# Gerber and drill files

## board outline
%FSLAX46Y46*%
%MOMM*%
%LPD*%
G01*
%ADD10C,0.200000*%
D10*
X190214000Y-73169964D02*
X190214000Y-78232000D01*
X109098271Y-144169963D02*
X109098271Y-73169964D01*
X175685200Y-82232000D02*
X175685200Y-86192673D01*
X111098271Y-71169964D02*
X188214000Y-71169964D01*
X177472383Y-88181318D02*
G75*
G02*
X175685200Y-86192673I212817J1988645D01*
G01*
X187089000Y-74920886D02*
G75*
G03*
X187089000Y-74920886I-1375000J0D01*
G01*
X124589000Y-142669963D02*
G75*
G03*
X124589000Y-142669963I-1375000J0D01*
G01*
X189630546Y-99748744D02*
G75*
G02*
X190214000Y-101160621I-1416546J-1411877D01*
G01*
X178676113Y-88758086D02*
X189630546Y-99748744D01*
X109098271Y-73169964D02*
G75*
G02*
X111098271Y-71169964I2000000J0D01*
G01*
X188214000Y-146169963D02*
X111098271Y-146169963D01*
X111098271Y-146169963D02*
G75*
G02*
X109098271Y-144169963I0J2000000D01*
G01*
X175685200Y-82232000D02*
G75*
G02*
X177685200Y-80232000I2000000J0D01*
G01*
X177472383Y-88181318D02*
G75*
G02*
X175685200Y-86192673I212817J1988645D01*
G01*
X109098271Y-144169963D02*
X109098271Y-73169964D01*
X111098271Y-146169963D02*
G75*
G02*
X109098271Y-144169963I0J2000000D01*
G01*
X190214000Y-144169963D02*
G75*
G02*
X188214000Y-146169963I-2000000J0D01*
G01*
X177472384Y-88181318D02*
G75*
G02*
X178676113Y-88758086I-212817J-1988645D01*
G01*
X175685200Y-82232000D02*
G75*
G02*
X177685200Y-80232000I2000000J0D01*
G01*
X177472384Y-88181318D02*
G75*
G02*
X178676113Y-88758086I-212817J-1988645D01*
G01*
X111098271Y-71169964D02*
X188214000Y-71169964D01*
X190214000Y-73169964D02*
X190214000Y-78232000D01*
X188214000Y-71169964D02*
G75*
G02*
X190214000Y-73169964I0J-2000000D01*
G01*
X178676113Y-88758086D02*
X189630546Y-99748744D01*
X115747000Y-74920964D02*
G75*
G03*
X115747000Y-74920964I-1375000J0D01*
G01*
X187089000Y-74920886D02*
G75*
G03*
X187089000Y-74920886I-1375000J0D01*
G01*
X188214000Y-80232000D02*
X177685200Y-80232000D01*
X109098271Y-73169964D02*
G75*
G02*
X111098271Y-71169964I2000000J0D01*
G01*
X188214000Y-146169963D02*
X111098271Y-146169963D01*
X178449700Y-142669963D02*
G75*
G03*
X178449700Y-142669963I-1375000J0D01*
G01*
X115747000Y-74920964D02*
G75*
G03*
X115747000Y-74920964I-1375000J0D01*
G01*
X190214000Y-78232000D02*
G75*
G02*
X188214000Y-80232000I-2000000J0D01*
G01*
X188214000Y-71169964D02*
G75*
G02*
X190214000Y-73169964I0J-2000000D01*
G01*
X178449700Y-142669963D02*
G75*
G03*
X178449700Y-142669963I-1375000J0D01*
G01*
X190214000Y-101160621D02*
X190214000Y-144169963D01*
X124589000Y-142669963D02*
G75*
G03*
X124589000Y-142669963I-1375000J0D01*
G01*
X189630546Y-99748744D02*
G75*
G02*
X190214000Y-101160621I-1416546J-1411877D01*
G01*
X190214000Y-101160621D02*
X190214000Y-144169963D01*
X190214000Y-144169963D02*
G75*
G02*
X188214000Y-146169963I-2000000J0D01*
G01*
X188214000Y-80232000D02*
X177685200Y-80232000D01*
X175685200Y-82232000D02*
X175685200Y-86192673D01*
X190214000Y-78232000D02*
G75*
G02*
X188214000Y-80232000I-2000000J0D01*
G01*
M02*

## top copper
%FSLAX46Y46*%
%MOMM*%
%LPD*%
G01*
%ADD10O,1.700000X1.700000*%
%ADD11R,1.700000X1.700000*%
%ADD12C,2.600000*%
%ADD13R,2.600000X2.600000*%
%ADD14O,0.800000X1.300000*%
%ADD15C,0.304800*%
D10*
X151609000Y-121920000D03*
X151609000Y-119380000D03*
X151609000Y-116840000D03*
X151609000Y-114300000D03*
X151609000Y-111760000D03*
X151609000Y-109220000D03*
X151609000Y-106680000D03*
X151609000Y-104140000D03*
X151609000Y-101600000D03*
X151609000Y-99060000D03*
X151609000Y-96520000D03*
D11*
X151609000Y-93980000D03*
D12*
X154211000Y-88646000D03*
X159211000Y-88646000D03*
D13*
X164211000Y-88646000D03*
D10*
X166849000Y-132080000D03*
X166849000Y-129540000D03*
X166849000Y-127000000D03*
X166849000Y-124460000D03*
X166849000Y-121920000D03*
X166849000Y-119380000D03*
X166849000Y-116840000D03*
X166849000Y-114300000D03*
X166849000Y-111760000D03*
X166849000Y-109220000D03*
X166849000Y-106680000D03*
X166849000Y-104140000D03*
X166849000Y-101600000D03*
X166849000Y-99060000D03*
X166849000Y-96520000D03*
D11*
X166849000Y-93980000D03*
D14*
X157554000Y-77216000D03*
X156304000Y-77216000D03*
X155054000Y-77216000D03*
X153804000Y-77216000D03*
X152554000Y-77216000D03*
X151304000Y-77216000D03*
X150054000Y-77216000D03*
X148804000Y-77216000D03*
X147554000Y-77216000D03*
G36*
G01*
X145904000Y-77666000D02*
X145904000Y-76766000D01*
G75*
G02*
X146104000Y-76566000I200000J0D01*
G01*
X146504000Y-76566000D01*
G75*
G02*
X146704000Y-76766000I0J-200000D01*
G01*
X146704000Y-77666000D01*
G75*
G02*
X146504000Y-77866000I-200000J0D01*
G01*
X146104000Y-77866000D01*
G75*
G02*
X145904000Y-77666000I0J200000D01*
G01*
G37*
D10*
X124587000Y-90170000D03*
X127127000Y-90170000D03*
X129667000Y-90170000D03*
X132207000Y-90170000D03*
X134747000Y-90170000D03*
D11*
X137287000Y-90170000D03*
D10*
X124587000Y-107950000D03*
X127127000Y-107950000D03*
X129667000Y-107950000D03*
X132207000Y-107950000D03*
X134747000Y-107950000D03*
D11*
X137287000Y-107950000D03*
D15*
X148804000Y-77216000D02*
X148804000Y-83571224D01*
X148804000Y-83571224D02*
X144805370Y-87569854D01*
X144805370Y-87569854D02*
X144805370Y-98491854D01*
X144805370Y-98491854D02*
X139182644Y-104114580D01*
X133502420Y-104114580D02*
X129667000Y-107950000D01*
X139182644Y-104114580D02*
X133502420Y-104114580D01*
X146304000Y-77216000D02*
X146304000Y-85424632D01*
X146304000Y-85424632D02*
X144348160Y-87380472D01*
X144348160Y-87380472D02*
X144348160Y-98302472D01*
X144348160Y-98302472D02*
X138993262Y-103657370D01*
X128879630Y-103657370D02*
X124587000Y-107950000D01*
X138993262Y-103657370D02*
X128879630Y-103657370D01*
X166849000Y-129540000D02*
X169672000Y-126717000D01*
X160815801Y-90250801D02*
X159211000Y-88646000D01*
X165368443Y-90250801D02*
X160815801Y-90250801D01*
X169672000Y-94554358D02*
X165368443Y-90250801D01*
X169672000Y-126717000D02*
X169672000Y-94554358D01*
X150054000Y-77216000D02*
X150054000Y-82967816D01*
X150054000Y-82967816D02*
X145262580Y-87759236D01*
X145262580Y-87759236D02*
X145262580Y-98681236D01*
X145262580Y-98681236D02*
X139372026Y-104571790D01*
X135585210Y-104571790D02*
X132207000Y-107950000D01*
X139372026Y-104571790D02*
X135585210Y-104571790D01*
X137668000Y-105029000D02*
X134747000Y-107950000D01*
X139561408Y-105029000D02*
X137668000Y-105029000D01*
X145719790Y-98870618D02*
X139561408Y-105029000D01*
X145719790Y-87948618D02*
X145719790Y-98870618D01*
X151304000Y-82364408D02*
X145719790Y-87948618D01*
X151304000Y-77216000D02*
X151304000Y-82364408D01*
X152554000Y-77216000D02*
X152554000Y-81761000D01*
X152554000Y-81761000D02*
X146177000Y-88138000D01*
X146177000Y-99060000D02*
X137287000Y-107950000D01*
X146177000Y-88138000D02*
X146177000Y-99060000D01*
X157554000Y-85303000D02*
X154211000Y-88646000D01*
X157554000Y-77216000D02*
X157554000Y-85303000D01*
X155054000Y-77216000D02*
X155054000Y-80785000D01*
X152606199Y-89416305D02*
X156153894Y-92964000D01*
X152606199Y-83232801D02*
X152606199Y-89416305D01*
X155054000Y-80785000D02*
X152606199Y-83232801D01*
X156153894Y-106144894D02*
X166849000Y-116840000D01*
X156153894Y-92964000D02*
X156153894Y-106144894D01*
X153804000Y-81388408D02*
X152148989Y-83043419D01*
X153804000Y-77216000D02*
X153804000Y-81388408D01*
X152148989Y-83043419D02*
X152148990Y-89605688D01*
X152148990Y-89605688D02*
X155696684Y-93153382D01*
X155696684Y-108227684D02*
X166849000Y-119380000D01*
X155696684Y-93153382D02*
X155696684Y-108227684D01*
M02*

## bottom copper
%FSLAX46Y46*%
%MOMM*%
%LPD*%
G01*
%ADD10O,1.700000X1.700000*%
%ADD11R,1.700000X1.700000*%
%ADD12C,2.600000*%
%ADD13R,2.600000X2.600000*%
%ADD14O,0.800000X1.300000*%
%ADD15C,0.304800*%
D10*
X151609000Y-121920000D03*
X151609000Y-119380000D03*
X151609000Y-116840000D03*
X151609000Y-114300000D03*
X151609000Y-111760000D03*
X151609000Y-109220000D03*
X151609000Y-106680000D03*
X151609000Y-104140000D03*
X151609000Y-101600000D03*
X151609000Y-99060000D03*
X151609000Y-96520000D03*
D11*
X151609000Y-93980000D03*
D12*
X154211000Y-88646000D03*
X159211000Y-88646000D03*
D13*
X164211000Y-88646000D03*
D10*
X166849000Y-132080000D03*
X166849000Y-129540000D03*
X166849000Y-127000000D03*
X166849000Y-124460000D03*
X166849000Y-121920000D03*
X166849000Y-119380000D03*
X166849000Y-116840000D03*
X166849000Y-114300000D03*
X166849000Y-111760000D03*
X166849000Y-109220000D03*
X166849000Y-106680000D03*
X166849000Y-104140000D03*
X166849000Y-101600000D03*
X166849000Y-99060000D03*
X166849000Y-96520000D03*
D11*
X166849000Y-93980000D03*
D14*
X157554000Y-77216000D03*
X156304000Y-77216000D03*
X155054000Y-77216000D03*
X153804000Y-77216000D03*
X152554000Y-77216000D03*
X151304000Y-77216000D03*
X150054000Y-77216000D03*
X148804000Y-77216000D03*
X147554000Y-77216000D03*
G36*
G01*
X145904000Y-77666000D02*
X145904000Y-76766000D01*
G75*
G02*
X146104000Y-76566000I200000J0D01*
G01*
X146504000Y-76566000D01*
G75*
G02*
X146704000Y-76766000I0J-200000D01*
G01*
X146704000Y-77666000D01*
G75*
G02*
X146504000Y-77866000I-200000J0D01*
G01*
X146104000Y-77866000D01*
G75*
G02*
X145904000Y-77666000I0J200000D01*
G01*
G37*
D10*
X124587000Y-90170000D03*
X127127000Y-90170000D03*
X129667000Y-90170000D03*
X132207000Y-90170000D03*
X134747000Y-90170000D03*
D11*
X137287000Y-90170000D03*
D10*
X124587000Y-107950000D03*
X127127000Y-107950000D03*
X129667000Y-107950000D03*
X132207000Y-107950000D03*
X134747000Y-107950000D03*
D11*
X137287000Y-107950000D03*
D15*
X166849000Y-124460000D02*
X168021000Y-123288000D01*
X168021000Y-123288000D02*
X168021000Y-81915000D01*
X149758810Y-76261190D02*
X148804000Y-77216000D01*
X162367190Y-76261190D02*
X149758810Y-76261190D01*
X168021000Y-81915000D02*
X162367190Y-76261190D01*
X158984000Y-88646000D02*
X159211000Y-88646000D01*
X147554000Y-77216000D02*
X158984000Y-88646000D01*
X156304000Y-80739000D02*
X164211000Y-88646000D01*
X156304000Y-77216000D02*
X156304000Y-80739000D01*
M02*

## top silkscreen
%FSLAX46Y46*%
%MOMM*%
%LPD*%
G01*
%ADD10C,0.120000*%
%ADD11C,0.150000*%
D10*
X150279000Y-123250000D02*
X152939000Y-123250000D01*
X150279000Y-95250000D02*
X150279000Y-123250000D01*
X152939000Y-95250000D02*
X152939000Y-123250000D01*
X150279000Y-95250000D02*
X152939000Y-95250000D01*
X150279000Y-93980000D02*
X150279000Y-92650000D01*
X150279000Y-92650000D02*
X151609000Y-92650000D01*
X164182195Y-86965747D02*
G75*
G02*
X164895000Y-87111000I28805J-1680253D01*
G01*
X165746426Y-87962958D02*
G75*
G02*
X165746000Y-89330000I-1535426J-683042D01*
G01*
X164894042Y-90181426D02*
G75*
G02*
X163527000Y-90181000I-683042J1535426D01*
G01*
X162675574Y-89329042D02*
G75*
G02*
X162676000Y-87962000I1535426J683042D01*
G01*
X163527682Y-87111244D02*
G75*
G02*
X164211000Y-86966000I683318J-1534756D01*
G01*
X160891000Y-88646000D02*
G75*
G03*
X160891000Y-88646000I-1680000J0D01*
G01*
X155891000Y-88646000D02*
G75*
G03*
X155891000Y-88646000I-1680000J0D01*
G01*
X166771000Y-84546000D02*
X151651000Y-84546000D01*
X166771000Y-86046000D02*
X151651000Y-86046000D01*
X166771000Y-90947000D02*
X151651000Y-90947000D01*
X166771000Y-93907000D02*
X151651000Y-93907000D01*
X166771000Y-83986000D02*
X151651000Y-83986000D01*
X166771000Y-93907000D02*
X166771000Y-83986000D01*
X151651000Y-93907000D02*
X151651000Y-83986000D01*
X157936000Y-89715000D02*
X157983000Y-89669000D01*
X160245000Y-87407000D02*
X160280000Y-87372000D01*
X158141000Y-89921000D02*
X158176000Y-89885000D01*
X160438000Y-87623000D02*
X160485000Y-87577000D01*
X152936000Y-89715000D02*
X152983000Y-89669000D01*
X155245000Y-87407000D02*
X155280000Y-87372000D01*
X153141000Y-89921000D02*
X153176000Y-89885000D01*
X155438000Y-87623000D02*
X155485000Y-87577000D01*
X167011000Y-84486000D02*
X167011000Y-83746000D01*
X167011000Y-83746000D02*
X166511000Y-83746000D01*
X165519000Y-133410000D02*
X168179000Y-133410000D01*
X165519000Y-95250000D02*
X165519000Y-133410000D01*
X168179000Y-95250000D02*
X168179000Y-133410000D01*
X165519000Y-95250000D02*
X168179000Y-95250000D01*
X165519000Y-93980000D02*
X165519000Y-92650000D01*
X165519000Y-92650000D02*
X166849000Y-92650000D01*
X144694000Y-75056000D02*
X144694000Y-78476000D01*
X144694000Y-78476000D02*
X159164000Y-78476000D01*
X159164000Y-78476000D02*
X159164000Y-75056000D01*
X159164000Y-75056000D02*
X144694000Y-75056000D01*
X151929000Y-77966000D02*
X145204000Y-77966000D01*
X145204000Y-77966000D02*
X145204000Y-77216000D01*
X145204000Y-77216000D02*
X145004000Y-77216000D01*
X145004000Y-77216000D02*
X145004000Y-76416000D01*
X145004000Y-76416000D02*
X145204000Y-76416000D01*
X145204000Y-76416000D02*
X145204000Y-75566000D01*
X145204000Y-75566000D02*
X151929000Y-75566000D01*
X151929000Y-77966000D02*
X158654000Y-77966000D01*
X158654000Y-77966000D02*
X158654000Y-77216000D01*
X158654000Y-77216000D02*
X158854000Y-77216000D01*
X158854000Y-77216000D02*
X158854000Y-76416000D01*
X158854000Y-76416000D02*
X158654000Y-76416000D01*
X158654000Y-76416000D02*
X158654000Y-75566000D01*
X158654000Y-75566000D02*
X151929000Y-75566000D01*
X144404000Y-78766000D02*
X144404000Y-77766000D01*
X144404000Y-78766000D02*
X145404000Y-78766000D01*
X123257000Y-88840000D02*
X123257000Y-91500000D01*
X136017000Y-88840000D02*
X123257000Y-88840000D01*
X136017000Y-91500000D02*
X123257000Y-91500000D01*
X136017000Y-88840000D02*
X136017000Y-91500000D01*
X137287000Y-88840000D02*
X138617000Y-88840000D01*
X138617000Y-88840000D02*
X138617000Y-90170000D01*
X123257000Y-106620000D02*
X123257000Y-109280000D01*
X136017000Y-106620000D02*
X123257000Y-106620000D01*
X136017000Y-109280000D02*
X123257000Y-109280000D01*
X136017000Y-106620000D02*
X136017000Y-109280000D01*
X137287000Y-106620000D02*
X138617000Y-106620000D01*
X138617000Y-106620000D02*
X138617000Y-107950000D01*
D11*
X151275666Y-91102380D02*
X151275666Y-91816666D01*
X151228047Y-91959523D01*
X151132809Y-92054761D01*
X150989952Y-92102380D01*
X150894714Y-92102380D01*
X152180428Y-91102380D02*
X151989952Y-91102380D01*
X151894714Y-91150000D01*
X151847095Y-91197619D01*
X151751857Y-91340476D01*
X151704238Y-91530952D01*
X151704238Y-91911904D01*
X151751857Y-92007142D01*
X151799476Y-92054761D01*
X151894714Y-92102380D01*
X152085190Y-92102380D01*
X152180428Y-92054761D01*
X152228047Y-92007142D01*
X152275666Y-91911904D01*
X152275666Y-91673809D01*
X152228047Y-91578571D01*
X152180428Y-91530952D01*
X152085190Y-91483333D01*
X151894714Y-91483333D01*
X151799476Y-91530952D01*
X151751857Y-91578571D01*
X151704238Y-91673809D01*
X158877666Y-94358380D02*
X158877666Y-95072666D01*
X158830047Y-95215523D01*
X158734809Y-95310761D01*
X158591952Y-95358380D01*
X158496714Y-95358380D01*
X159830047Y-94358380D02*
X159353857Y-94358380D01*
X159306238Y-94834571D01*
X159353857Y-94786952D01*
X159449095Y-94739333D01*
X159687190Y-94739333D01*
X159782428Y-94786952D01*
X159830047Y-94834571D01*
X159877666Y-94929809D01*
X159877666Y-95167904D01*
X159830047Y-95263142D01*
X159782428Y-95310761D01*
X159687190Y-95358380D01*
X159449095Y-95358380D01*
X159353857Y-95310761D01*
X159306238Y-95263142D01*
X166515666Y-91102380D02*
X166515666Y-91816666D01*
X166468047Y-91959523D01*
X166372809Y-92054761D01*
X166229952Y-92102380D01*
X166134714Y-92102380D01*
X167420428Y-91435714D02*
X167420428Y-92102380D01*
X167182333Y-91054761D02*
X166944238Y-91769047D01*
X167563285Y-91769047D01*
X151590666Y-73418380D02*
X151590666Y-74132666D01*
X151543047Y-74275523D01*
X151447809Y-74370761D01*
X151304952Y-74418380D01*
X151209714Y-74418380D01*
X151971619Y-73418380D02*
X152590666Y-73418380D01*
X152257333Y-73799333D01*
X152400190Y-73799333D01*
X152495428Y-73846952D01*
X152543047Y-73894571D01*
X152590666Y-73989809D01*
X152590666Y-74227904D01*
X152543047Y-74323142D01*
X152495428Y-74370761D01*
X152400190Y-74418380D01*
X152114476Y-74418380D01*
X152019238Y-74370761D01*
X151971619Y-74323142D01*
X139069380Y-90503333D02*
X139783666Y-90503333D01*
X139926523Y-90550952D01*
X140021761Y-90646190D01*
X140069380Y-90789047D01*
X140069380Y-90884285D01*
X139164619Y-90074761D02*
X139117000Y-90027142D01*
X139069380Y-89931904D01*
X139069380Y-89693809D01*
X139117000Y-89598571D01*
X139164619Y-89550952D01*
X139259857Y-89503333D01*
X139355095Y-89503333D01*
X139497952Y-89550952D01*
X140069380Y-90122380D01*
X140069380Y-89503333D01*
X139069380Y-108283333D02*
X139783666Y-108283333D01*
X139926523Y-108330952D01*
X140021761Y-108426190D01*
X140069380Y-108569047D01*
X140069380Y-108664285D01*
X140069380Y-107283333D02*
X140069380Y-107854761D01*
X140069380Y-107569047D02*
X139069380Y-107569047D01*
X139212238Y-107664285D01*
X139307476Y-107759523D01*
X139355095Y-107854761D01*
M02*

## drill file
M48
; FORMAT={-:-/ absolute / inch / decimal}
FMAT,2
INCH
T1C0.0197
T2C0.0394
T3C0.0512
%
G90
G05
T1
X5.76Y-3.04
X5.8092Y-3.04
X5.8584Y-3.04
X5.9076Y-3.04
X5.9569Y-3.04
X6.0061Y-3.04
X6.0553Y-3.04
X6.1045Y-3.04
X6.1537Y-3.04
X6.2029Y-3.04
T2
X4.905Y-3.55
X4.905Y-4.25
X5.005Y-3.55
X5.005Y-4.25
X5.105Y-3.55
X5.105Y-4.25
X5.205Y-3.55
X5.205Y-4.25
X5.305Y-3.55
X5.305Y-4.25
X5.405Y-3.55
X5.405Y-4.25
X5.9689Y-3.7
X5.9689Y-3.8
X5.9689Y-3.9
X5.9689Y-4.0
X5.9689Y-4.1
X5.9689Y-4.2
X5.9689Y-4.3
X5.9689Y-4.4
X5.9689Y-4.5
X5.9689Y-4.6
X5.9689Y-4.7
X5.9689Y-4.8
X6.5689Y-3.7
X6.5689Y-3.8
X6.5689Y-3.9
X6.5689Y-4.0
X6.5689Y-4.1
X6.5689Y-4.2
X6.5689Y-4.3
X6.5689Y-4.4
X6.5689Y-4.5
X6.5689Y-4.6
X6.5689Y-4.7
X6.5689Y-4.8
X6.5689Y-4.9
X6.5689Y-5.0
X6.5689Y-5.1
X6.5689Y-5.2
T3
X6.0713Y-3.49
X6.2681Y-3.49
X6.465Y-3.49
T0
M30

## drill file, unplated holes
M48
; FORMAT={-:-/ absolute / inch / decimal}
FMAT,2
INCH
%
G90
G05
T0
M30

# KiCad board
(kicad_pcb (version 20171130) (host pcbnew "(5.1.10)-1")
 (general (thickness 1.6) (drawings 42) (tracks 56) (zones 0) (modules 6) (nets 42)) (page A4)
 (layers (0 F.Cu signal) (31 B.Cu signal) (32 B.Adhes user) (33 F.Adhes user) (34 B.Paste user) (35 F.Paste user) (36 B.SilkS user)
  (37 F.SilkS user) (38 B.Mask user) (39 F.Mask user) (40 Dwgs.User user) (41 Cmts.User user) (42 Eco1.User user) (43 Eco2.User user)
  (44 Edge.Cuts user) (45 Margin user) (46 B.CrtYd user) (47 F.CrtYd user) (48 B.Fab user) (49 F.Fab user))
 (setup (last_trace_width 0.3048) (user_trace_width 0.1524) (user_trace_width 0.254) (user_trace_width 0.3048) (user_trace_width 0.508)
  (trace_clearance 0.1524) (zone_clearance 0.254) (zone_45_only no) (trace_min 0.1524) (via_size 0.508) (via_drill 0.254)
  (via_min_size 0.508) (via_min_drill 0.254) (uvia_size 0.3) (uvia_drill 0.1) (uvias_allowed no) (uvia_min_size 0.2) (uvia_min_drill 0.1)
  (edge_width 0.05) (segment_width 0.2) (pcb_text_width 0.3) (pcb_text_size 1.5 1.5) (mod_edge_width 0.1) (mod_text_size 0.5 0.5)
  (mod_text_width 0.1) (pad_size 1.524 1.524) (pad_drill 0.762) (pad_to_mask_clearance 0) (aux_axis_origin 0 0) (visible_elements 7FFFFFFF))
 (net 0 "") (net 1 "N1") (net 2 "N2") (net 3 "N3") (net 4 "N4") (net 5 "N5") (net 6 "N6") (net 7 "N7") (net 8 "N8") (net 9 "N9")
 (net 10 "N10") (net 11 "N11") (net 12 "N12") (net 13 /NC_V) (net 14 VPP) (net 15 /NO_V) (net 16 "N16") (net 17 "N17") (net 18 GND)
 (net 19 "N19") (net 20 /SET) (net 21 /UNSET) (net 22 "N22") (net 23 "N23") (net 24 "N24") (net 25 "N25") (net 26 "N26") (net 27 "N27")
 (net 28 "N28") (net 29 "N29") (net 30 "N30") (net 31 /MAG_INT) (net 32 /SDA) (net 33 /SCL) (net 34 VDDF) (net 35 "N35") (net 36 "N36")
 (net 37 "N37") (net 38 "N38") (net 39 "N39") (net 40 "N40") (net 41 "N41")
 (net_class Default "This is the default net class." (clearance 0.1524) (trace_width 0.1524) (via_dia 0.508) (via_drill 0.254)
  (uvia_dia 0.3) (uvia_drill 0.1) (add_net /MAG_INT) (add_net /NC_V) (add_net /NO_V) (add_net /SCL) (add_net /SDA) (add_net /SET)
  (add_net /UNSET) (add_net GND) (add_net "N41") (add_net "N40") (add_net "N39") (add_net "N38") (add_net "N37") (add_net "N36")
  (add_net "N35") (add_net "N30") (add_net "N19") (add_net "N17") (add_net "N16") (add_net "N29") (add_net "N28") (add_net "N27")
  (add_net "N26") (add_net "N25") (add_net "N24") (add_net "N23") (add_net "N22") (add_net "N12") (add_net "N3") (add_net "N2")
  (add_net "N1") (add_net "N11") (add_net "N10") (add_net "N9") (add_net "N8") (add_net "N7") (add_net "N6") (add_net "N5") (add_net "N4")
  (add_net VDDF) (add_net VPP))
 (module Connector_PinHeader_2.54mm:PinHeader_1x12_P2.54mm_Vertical (layer F.Cu) (at 151.609 93.98)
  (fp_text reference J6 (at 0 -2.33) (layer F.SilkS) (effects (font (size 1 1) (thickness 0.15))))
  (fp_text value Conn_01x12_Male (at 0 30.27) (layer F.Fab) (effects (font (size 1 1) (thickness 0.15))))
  (fp_line (start -1.33 29.27) (end 1.33 29.27) (layer F.SilkS) (width 0.12))
  (fp_line (start -1.33 1.27) (end -1.33 29.27) (layer F.SilkS) (width 0.12))
  (fp_line (start 1.33 1.27) (end 1.33 29.27) (layer F.SilkS) (width 0.12))
  (fp_line (start -1.33 1.27) (end 1.33 1.27) (layer F.SilkS) (width 0.12))
  (fp_line (start -1.33 0) (end -1.33 -1.33) (layer F.SilkS) (width 0.12))
  (fp_line (start -1.33 -1.33) (end 0 -1.33) (layer F.SilkS) (width 0.12))
  (pad 12 thru_hole oval (at 0 27.94) (size 1.7 1.7) (drill 1) (layers *.Cu *.Mask) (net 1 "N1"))
  (pad 11 thru_hole oval (at 0 25.4) (size 1.7 1.7) (drill 1) (layers *.Cu *.Mask) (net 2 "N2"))
  (pad 10 thru_hole oval (at 0 22.86) (size 1.7 1.7) (drill 1) (layers *.Cu *.Mask) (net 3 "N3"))
  (pad 9 thru_hole oval (at 0 20.32) (size 1.7 1.7) (drill 1) (layers *.Cu *.Mask) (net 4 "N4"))
  (pad 8 thru_hole oval (at 0 17.78) (size 1.7 1.7) (drill 1) (layers *.Cu *.Mask) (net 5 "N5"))
  (pad 7 thru_hole oval (at 0 15.24) (size 1.7 1.7) (drill 1) (layers *.Cu *.Mask) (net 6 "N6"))
  (pad 6 thru_hole oval (at 0 12.7) (size 1.7 1.7) (drill 1) (layers *.Cu *.Mask) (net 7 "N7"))
  (pad 5 thru_hole oval (at 0 10.16) (size 1.7 1.7) (drill 1) (layers *.Cu *.Mask) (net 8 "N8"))
  (pad 4 thru_hole oval (at 0 7.62) (size 1.7 1.7) (drill 1) (layers *.Cu *.Mask) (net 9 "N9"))
  (pad 3 thru_hole oval (at 0 5.08) (size 1.7 1.7) (drill 1) (layers *.Cu *.Mask) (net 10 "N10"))
  (pad 2 thru_hole oval (at 0 2.54) (size 1.7 1.7) (drill 1) (layers *.Cu *.Mask) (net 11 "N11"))
  (pad 1 thru_hole rect (at 0 0) (size 1.7 1.7) (drill 1) (layers *.Cu *.Mask) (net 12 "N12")))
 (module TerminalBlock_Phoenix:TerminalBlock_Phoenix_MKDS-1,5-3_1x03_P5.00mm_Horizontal (layer F.Cu) (at 164.211 88.646 180)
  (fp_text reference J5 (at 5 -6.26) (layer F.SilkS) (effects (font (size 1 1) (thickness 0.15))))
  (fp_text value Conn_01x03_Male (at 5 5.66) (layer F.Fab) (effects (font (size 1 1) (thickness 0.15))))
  (fp_arc (start 0 0) (end -0.684 1.535) (angle -25) (layer F.SilkS) (width 0.12))
  (fp_arc (start 0 0) (end -1.535 -0.684) (angle -48) (layer F.SilkS) (width 0.12))
  (fp_arc (start 0 0) (end 0.684 -1.535) (angle -48) (layer F.SilkS) (width 0.12))
  (fp_arc (start 0 0) (end 1.535 0.684) (angle -48) (layer F.SilkS) (width 0.12))
  (fp_arc (start 0 0) (end 0 1.68) (angle -24) (layer F.SilkS) (width 0.12))
  (fp_circle (center 5 0) (end 6.68 0) (layer F.SilkS) (width 0.12))
  (fp_circle (center 10 0) (end 11.68 0) (layer F.SilkS) (width 0.12))
  (fp_line (start -2.56 4.1) (end 12.56 4.1) (layer F.SilkS) (width 0.12))
  (fp_line (start -2.56 2.6) (end 12.56 2.6) (layer F.SilkS) (width 0.12))
  (fp_line (start -2.56 -2.301) (end 12.56 -2.301) (layer F.SilkS) (width 0.12))
  (fp_line (start -2.56 -5.261) (end 12.56 -5.261) (layer F.SilkS) (width 0.12))
  (fp_line (start -2.56 4.66) (end 12.56 4.66) (layer F.SilkS) (width 0.12))
  (fp_line (start -2.56 -5.261) (end -2.56 4.66) (layer F.SilkS) (width 0.12))
  (fp_line (start 12.56 -5.261) (end 12.56 4.66) (layer F.SilkS) (width 0.12))
  (fp_line (start 6.275 -1.069) (end 6.228 -1.023) (layer F.SilkS) (width 0.12))
  (fp_line (start 3.966 1.239) (end 3.931 1.274) (layer F.SilkS) (width 0.12))
  (fp_line (start 6.07 -1.275) (end 6.035 -1.239) (layer F.SilkS) (width 0.12))
  (fp_line (start 3.773 1.023) (end 3.726 1.069) (layer F.SilkS) (width 0.12))
  (fp_line (start 11.275 -1.069) (end 11.228 -1.023) (layer F.SilkS) (width 0.12))
  (fp_line (start 8.966 1.239) (end 8.931 1.274) (layer F.SilkS) (width 0.12))
  (fp_line (start 11.07 -1.275) (end 11.035 -1.239) (layer F.SilkS) (width 0.12))
  (fp_line (start 8.773 1.023) (end 8.726 1.069) (layer F.SilkS) (width 0.12))
  (fp_line (start -2.8 4.16) (end -2.8 4.9) (layer F.SilkS) (width 0.12))
  (fp_line (start -2.8 4.9) (end -2.3 4.9) (layer F.SilkS) (width 0.12))
  (pad 3 thru_hole circle (at 10 0 180) (size 2.6 2.6) (drill 1.3) (layers *.Cu *.Mask) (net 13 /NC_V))
  (pad 2 thru_hole circle (at 5 0 180) (size 2.6 2.6) (drill 1.3) (layers *.Cu *.Mask) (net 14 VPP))
  (pad 1 thru_hole rect (at 0 0 180) (size 2.6 2.6) (drill 1.3) (layers *.Cu *.Mask) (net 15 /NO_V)))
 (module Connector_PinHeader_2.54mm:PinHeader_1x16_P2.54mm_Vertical (layer F.Cu) (at 166.849 93.98)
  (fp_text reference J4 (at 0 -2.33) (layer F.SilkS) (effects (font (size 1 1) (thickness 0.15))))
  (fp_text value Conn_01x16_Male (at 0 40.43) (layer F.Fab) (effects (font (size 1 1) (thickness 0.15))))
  (fp_line (start -1.33 39.43) (end 1.33 39.43) (layer F.SilkS) (width 0.12))
  (fp_line (start -1.33 1.27) (end -1.33 39.43) (layer F.SilkS) (width 0.12))
  (fp_line (start 1.33 1.27) (end 1.33 39.43) (layer F.SilkS) (width 0.12))
  (fp_line (start -1.33 1.27) (end 1.33 1.27) (layer F.SilkS) (width 0.12))
  (fp_line (start -1.33 0) (end -1.33 -1.33) (layer F.SilkS) (width 0.12))
  (fp_line (start -1.33 -1.33) (end 0 -1.33) (layer F.SilkS) (width 0.12))
  (pad 16 thru_hole oval (at 0 38.1) (size 1.7 1.7) (drill 1) (layers *.Cu *.Mask) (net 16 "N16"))
  (pad 15 thru_hole oval (at 0 35.56) (size 1.7 1.7) (drill 1) (layers *.Cu *.Mask) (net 14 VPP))
  (pad 14 thru_hole oval (at 0 33.02) (size 1.7 1.7) (drill 1) (layers *.Cu *.Mask) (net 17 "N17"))
  (pad 13 thru_hole oval (at 0 30.48) (size 1.7 1.7) (drill 1) (layers *.Cu *.Mask) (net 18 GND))
  (pad 12 thru_hole oval (at 0 27.94) (size 1.7 1.7) (drill 1) (layers *.Cu *.Mask) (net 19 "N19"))
  (pad 11 thru_hole oval (at 0 25.4) (size 1.7 1.7) (drill 1) (layers *.Cu *.Mask) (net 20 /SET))
  (pad 10 thru_hole oval (at 0 22.86) (size 1.7 1.7) (drill 1) (layers *.Cu *.Mask) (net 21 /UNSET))
  (pad 9 thru_hole oval (at 0 20.32) (size 1.7 1.7) (drill 1) (layers *.Cu *.Mask) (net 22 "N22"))
  (pad 8 thru_hole oval (at 0 17.78) (size 1.7 1.7) (drill 1) (layers *.Cu *.Mask) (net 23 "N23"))
  (pad 7 thru_hole oval (at 0 15.24) (size 1.7 1.7) (drill 1) (layers *.Cu *.Mask) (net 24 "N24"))
  (pad 6 thru_hole oval (at 0 12.7) (size 1.7 1.7) (drill 1) (layers *.Cu *.Mask) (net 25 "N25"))
  (pad 5 thru_hole oval (at 0 10.16) (size 1.7 1.7) (drill 1) (layers *.Cu *.Mask) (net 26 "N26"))
  (pad 4 thru_hole oval (at 0 7.62) (size 1.7 1.7) (drill 1) (layers *.Cu *.Mask) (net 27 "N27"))
  (pad 3 thru_hole oval (at 0 5.08) (size 1.7 1.7) (drill 1) (layers *.Cu *.Mask) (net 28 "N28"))
  (pad 2 thru_hole oval (at 0 2.54) (size 1.7 1.7) (drill 1) (layers *.Cu *.Mask) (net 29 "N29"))
  (pad 1 thru_hole rect (at 0 0) (size 1.7 1.7) (drill 1) (layers *.Cu *.Mask) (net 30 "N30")))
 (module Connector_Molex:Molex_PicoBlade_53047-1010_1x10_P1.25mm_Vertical (layer F.Cu) (at 146.304 77.216)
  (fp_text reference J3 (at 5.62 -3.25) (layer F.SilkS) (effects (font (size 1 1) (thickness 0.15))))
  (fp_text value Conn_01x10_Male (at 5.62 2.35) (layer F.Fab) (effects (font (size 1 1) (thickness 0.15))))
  (fp_line (start -1.61 -2.16) (end -1.61 1.26) (layer F.SilkS) (width 0.12))
  (fp_line (start -1.61 1.26) (end 12.86 1.26) (layer F.SilkS) (width 0.12))
  (fp_line (start 12.86 1.26) (end 12.86 -2.16) (layer F.SilkS) (width 0.12))
  (fp_line (start 12.86 -2.16) (end -1.61 -2.16) (layer F.SilkS) (width 0.12))
  (fp_line (start 5.625 0.75) (end -1.1 0.75) (layer F.SilkS) (width 0.12))
  (fp_line (start -1.1 0.75) (end -1.1 0) (layer F.SilkS) (width 0.12))
  (fp_line (start -1.1 0) (end -1.3 0) (layer F.SilkS) (width 0.12))
  (fp_line (start -1.3 0) (end -1.3 -0.8) (layer F.SilkS) (width 0.12))
  (fp_line (start -1.3 -0.8) (end -1.1 -0.8) (layer F.SilkS) (width 0.12))
  (fp_line (start -1.1 -0.8) (end -1.1 -1.65) (layer F.SilkS) (width 0.12))
  (fp_line (start -1.1 -1.65) (end 5.625 -1.65) (layer F.SilkS) (width 0.12))
  (fp_line (start 5.625 0.75) (end 12.35 0.75) (layer F.SilkS) (width 0.12))
  (fp_line (start 12.35 0.75) (end 12.35 0) (layer F.SilkS) (width 0.12))
  (fp_line (start 12.35 0) (end 12.55 0) (layer F.SilkS) (width 0.12))
  (fp_line (start 12.55 0) (end 12.55 -0.8) (layer F.SilkS) (width 0.12))
  (fp_line (start 12.55 -0.8) (end 12.35 -0.8) (layer F.SilkS) (width 0.12))
  (fp_line (start 12.35 -0.8) (end 12.35 -1.65) (layer F.SilkS) (width 0.12))
  (fp_line (start 12.35 -1.65) (end 5.625 -1.65) (layer F.SilkS) (width 0.12))
  (fp_line (start -1.9 1.55) (end -1.9 0.55) (layer F.SilkS) (width 0.12))
  (fp_line (start -1.9 1.55) (end -0.9 1.55) (layer F.SilkS) (width 0.12))
  (pad 10 thru_hole oval (at 11.25 0) (size 0.8 1.3) (drill 0.5) (layers *.Cu *.Mask) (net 13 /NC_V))
  (pad 9 thru_hole oval (at 10 0) (size 0.8 1.3) (drill 0.5) (layers *.Cu *.Mask) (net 15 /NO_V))
  (pad 8 thru_hole oval (at 8.75 0) (size 0.8 1.3) (drill 0.5) (layers *.Cu *.Mask) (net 21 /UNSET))
  (pad 7 thru_hole oval (at 7.5 0) (size 0.8 1.3) (drill 0.5) (layers *.Cu *.Mask) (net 20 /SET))
  (pad 6 thru_hole oval (at 6.25 0) (size 0.8 1.3) (drill 0.5) (layers *.Cu *.Mask) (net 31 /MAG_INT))
  (pad 5 thru_hole oval (at 5 0) (size 0.8 1.3) (drill 0.5) (layers *.Cu *.Mask) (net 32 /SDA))
  (pad 4 thru_hole oval (at 3.75 0) (size 0.8 1.3) (drill 0.5) (layers *.Cu *.Mask) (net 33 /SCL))
  (pad 3 thru_hole oval (at 2.5 0) (size 0.8 1.3) (drill 0.5) (layers *.Cu *.Mask) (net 18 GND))
  (pad 2 thru_hole oval (at 1.25 0) (size 0.8 1.3) (drill 0.5) (layers *.Cu *.Mask) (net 14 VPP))
  (pad 1 thru_hole roundrect (at 0 0) (size 0.8 1.3) (drill 0.5) (layers *.Cu *.Mask) (roundrect_rratio 0.25) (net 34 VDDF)))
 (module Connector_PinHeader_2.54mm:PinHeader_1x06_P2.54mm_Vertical (layer F.Cu) (at 137.287 90.17 270)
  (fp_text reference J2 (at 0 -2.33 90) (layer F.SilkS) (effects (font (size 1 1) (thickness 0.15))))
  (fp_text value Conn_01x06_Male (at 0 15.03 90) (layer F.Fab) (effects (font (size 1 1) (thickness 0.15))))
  (fp_line (start -1.33 14.03) (end 1.33 14.03) (layer F.SilkS) (width 0.12))
  (fp_line (start -1.33 1.27) (end -1.33 14.03) (layer F.SilkS) (width 0.12))
  (fp_line (start 1.33 1.27) (end 1.33 14.03) (layer F.SilkS) (width 0.12))
  (fp_line (start -1.33 1.27) (end 1.33 1.27) (layer F.SilkS) (width 0.12))
  (fp_line (start -1.33 0) (end -1.33 -1.33) (layer F.SilkS) (width 0.12))
  (fp_line (start -1.33 -1.33) (end 0 -1.33) (layer F.SilkS) (width 0.12))
  (pad 6 thru_hole oval (at 0 12.7 270) (size 1.7 1.7) (drill 1) (layers *.Cu *.Mask) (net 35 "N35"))
  (pad 5 thru_hole oval (at 0 10.16 270) (size 1.7 1.7) (drill 1) (layers *.Cu *.Mask) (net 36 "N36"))
  (pad 4 thru_hole oval (at 0 7.62 270) (size 1.7 1.7) (drill 1) (layers *.Cu *.Mask) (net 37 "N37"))
  (pad 3 thru_hole oval (at 0 5.08 270) (size 1.7 1.7) (drill 1) (layers *.Cu *.Mask) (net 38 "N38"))
  (pad 2 thru_hole oval (at 0 2.54 270) (size 1.7 1.7) (drill 1) (layers *.Cu *.Mask) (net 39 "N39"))
  (pad 1 thru_hole rect (at 0 0 270) (size 1.7 1.7) (drill 1) (layers *.Cu *.Mask) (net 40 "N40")))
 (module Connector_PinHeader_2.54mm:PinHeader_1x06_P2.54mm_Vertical (layer F.Cu) (at 137.287 107.95 270)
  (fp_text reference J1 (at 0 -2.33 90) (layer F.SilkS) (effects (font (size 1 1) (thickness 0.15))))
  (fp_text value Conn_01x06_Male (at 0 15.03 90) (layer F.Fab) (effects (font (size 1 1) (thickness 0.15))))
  (fp_line (start -1.33 14.03) (end 1.33 14.03) (layer F.SilkS) (width 0.12))
  (fp_line (start -1.33 1.27) (end -1.33 14.03) (layer F.SilkS) (width 0.12))
  (fp_line (start 1.33 1.27) (end 1.33 14.03) (layer F.SilkS) (width 0.12))
  (fp_line (start -1.33 1.27) (end 1.33 1.27) (layer F.SilkS) (width 0.12))
  (fp_line (start -1.33 0) (end -1.33 -1.33) (layer F.SilkS) (width 0.12))
  (fp_line (start -1.33 -1.33) (end 0 -1.33) (layer F.SilkS) (width 0.12))
  (pad 6 thru_hole oval (at 0 12.7 270) (size 1.7 1.7) (drill 1) (layers *.Cu *.Mask) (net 34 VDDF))
  (pad 5 thru_hole oval (at 0 10.16 270) (size 1.7 1.7) (drill 1) (layers *.Cu *.Mask) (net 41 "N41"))
  (pad 4 thru_hole oval (at 0 7.62 270) (size 1.7 1.7) (drill 1) (layers *.Cu *.Mask) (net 18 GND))
  (pad 3 thru_hole oval (at 0 5.08 270) (size 1.7 1.7) (drill 1) (layers *.Cu *.Mask) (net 33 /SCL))
  (pad 2 thru_hole oval (at 0 2.54 270) (size 1.7 1.7) (drill 1) (layers *.Cu *.Mask) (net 32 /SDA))
  (pad 1 thru_hole rect (at 0 0 270) (size 1.7 1.7) (drill 1) (layers *.Cu *.Mask) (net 31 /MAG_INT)))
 (gr_line (start 190.214 73.169964) (end 190.214 78.232) (layer Edge.Cuts) (width 0.2))
 (gr_line (start 109.098271 144.169963) (end 109.098271 73.169964) (layer Edge.Cuts) (width 0.2))
 (gr_line (start 175.6852 82.232) (end 175.6852 86.192673) (layer Edge.Cuts) (width 0.2))
 (gr_line (start 111.098271 71.169964) (end 188.214 71.169964) (layer Edge.Cuts) (width 0.2))
 (gr_arc (start 177.6852 86.192673) (end 175.6852 86.192673) (angle -83.89169034) (layer Edge.Cuts) (width 0.2))
 (gr_circle (center 185.714 74.920886) (end 187.089 74.920886) (layer Edge.Cuts) (width 0.2))
 (gr_circle (center 123.214 142.669963) (end 124.589 142.669963) (layer Edge.Cuts) (width 0.2))
 (gr_arc (start 188.214 101.160621) (end 190.214 101.160621) (angle -44.90542239) (layer Edge.Cuts) (width 0.2))
 (gr_line (start 178.676113 88.758086) (end 189.630546 99.748744) (layer Edge.Cuts) (width 0.2))
 (gr_arc (start 111.098271 73.169964) (end 111.098271 71.169964) (angle -90) (layer Edge.Cuts) (width 0.2))
 (gr_line (start 188.214 146.169963) (end 111.098271 146.169963) (layer Edge.Cuts) (width 0.2))
 (gr_arc (start 111.098271 144.169963) (end 109.098271 144.169963) (angle -90) (layer Edge.Cuts) (width 0.2))
 (gr_arc (start 177.6852 82.232) (end 177.6852 80.232) (angle -90) (layer Edge.Cuts) (width 0.2))
 (gr_arc (start 177.6852 86.192673) (end 175.6852 86.192673) (angle -83.89169034) (layer Edge.Cuts) (width 0.2))
 (gr_line (start 109.098271 144.169963) (end 109.098271 73.169964) (layer Edge.Cuts) (width 0.2))
 (gr_arc (start 111.098271 144.169963) (end 109.098271 144.169963) (angle -90) (layer Edge.Cuts) (width 0.2))
 (gr_arc (start 188.214 144.169963) (end 188.214 146.169963) (angle -90) (layer Edge.Cuts) (width 0.2))
 (gr_arc (start 177.259567 90.169963) (end 178.676113 88.758086) (angle -38.98626795) (layer Edge.Cuts) (width 0.2))
 (gr_arc (start 177.6852 82.232) (end 177.6852 80.232) (angle -90) (layer Edge.Cuts) (width 0.2))
 (gr_arc (start 177.259567 90.169963) (end 178.676113 88.758086) (angle -38.98626795) (layer Edge.Cuts) (width 0.2))
 (gr_line (start 111.098271 71.169964) (end 188.214 71.169964) (layer Edge.Cuts) (width 0.2))
 (gr_line (start 190.214 73.169964) (end 190.214 78.232) (layer Edge.Cuts) (width 0.2))
 (gr_arc (start 188.214 73.169964) (end 190.214 73.169964) (angle -90) (layer Edge.Cuts) (width 0.2))
 (gr_line (start 178.676113 88.758086) (end 189.630546 99.748744) (layer Edge.Cuts) (width 0.2))
 (gr_circle (center 114.372 74.920964) (end 115.747 74.920964) (layer Edge.Cuts) (width 0.2))
 (gr_circle (center 185.714 74.920886) (end 187.089 74.920886) (layer Edge.Cuts) (width 0.2))
 (gr_line (start 188.214 80.232) (end 177.6852 80.232) (layer Edge.Cuts) (width 0.2))
 (gr_arc (start 111.098271 73.169964) (end 111.098271 71.169964) (angle -90) (layer Edge.Cuts) (width 0.2))
 (gr_line (start 188.214 146.169963) (end 111.098271 146.169963) (layer Edge.Cuts) (width 0.2))
 (gr_circle (center 177.0747 142.669963) (end 178.4497 142.669963) (layer Edge.Cuts) (width 0.2))
 (gr_circle (center 114.372 74.920964) (end 115.747 74.920964) (layer Edge.Cuts) (width 0.2))
 (gr_arc (start 188.214 78.232) (end 188.214 80.232) (angle -90) (layer Edge.Cuts) (width 0.2))
 (gr_arc (start 188.214 73.169964) (end 190.214 73.169964) (angle -90) (layer Edge.Cuts) (width 0.2))
 (gr_circle (center 177.0747 142.669963) (end 178.4497 142.669963) (layer Edge.Cuts) (width 0.2))
 (gr_line (start 190.214 101.160621) (end 190.214 144.169963) (layer Edge.Cuts) (width 0.2))
 (gr_circle (center 123.214 142.669963) (end 124.589 142.669963) (layer Edge.Cuts) (width 0.2))
 (gr_arc (start 188.214 101.160621) (end 190.214 101.160621) (angle -44.90542239) (layer Edge.Cuts) (width 0.2))
 (gr_line (start 190.214 101.160621) (end 190.214 144.169963) (layer Edge.Cuts) (width 0.2))
 (gr_arc (start 188.214 144.169963) (end 188.214 146.169963) (angle -90) (layer Edge.Cuts) (width 0.2))
 (gr_line (start 188.214 80.232) (end 177.6852 80.232) (layer Edge.Cuts) (width 0.2))
 (gr_line (start 175.6852 82.232) (end 175.6852 86.192673) (layer Edge.Cuts) (width 0.2))
 (gr_arc (start 188.214 78.232) (end 188.214 80.232) (angle -90) (layer Edge.Cuts) (width 0.2))
 (segment (start 148.804 77.216) (end 148.804 83.571224) (width 0.3048) (layer F.Cu) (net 18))
 (segment (start 148.804 83.571224) (end 144.80537 87.569854) (width 0.3048) (layer F.Cu) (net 18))
 (segment (start 144.80537 87.569854) (end 144.80537 98.491854) (width 0.3048) (layer F.Cu) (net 18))
 (segment (start 144.80537 98.491854) (end 139.182644 104.11458) (width 0.3048) (layer F.Cu) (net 18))
 (segment (start 133.50242 104.11458) (end 129.667 107.95) (width 0.3048) (layer F.Cu) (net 18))
 (segment (start 139.182644 104.11458) (end 133.50242 104.11458) (width 0.3048) (layer F.Cu) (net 18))
 (segment (start 166.849 124.46) (end 168.021 123.288) (width 0.3048) (layer B.Cu) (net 18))
 (segment (start 168.021 123.288) (end 168.021 81.915) (width 0.3048) (layer B.Cu) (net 18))
 (segment (start 149.75881 76.26119) (end 148.804 77.216) (width 0.3048) (layer B.Cu) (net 18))
 (segment (start 162.36719 76.26119) (end 149.75881 76.26119) (width 0.3048) (layer B.Cu) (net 18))
 (segment (start 168.021 81.915) (end 162.36719 76.26119) (width 0.3048) (layer B.Cu) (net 18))
 (segment (start 146.304 77.216) (end 146.304 85.424632) (width 0.3048) (layer F.Cu) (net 34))
 (segment (start 146.304 85.424632) (end 144.34816 87.380472) (width 0.3048) (layer F.Cu) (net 34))
 (segment (start 144.34816 87.380472) (end 144.34816 98.302472) (width 0.3048) (layer F.Cu) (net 34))
 (segment (start 144.34816 98.302472) (end 138.993262 103.65737) (width 0.3048) (layer F.Cu) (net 34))
 (segment (start 128.87963 103.65737) (end 124.587 107.95) (width 0.3048) (layer F.Cu) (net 34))
 (segment (start 138.993262 103.65737) (end 128.87963 103.65737) (width 0.3048) (layer F.Cu) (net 34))
 (segment (start 158.984 88.646) (end 159.211 88.646) (width 0.3048) (layer B.Cu) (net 14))
 (segment (start 147.554 77.216) (end 158.984 88.646) (width 0.3048) (layer B.Cu) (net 14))
 (segment (start 166.849 129.54) (end 169.672 126.717) (width 0.3048) (layer F.Cu) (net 14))
 (segment (start 160.815801 90.250801) (end 159.211 88.646) (width 0.3048) (layer F.Cu) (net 14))
 (segment (start 165.368443 90.250801) (end 160.815801 90.250801) (width 0.3048) (layer F.Cu) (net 14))
 (segment (start 169.672 94.554358) (end 165.368443 90.250801) (width 0.3048) (layer F.Cu) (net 14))
 (segment (start 169.672 126.717) (end 169.672 94.554358) (width 0.3048) (layer F.Cu) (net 14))
 (segment (start 150.054 77.216) (end 150.054 82.967816) (width 0.3048) (layer F.Cu) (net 33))
 (segment (start 150.054 82.967816) (end 145.26258 87.759236) (width 0.3048) (layer F.Cu) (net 33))
 (segment (start 145.26258 87.759236) (end 145.26258 98.681236) (width 0.3048) (layer F.Cu) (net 33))
 (segment (start 145.26258 98.681236) (end 139.372026 104.57179) (width 0.3048) (layer F.Cu) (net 33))
 (segment (start 135.58521 104.57179) (end 132.207 107.95) (width 0.3048) (layer F.Cu) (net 33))
 (segment (start 139.372026 104.57179) (end 135.58521 104.57179) (width 0.3048) (layer F.Cu) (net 33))
 (segment (start 137.668 105.029) (end 134.747 107.95) (width 0.3048) (layer F.Cu) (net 32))
 (segment (start 139.561408 105.029) (end 137.668 105.029) (width 0.3048) (layer F.Cu) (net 32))
 (segment (start 145.71979 98.870618) (end 139.561408 105.029) (width 0.3048) (layer F.Cu) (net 32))
 (segment (start 145.71979 87.948618) (end 145.71979 98.870618) (width 0.3048) (layer F.Cu) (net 32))
 (segment (start 151.304 82.364408) (end 145.71979 87.948618) (width 0.3048) (layer F.Cu) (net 32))
 (segment (start 151.304 77.216) (end 151.304 82.364408) (width 0.3048) (layer F.Cu) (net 32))
 (segment (start 152.554 77.216) (end 152.554 81.761) (width 0.3048) (layer F.Cu) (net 31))
 (segment (start 152.554 81.761) (end 146.177 88.138) (width 0.3048) (layer F.Cu) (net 31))
 (segment (start 146.177 99.06) (end 137.287 107.95) (width 0.3048) (layer F.Cu) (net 31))
 (segment (start 146.177 88.138) (end 146.177 99.06) (width 0.3048) (layer F.Cu) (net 31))
 (segment (start 157.554 85.303) (end 154.211 88.646) (width 0.3048) (layer F.Cu) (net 13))
 (segment (start 157.554 77.216) (end 157.554 85.303) (width 0.3048) (layer F.Cu) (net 13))
 (segment (start 156.304 80.739) (end 164.211 88.646) (width 0.3048) (layer B.Cu) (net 15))
 (segment (start 156.304 77.216) (end 156.304 80.739) (width 0.3048) (layer B.Cu) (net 15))
 (segment (start 155.054 77.216) (end 155.054 80.785) (width 0.3048) (layer F.Cu) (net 21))
 (segment (start 152.606199 89.416305) (end 156.153894 92.964) (width 0.3048) (layer F.Cu) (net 21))
 (segment (start 152.606199 83.232801) (end 152.606199 89.416305) (width 0.3048) (layer F.Cu) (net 21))
 (segment (start 155.054 80.785) (end 152.606199 83.232801) (width 0.3048) (layer F.Cu) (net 21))
 (segment (start 156.153894 106.144894) (end 166.849 116.84) (width 0.3048) (layer F.Cu) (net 21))
 (segment (start 156.153894 92.964) (end 156.153894 106.144894) (width 0.3048) (layer F.Cu) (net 21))
 (segment (start 153.804 81.388408) (end 152.148989 83.043419) (width 0.3048) (layer F.Cu) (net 20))
 (segment (start 153.804 77.216) (end 153.804 81.388408) (width 0.3048) (layer F.Cu) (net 20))
 (segment (start 152.148989 83.043419) (end 152.14899 89.605688) (width 0.3048) (layer F.Cu) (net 20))
 (segment (start 152.14899 89.605688) (end 155.696684 93.153382) (width 0.3048) (layer F.Cu) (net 20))
 (segment (start 155.696684 108.227684) (end 166.849 119.38) (width 0.3048) (layer F.Cu) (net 20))
 (segment (start 155.696684 93.153382) (end 155.696684 108.227684) (width 0.3048) (layer F.Cu) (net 20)))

